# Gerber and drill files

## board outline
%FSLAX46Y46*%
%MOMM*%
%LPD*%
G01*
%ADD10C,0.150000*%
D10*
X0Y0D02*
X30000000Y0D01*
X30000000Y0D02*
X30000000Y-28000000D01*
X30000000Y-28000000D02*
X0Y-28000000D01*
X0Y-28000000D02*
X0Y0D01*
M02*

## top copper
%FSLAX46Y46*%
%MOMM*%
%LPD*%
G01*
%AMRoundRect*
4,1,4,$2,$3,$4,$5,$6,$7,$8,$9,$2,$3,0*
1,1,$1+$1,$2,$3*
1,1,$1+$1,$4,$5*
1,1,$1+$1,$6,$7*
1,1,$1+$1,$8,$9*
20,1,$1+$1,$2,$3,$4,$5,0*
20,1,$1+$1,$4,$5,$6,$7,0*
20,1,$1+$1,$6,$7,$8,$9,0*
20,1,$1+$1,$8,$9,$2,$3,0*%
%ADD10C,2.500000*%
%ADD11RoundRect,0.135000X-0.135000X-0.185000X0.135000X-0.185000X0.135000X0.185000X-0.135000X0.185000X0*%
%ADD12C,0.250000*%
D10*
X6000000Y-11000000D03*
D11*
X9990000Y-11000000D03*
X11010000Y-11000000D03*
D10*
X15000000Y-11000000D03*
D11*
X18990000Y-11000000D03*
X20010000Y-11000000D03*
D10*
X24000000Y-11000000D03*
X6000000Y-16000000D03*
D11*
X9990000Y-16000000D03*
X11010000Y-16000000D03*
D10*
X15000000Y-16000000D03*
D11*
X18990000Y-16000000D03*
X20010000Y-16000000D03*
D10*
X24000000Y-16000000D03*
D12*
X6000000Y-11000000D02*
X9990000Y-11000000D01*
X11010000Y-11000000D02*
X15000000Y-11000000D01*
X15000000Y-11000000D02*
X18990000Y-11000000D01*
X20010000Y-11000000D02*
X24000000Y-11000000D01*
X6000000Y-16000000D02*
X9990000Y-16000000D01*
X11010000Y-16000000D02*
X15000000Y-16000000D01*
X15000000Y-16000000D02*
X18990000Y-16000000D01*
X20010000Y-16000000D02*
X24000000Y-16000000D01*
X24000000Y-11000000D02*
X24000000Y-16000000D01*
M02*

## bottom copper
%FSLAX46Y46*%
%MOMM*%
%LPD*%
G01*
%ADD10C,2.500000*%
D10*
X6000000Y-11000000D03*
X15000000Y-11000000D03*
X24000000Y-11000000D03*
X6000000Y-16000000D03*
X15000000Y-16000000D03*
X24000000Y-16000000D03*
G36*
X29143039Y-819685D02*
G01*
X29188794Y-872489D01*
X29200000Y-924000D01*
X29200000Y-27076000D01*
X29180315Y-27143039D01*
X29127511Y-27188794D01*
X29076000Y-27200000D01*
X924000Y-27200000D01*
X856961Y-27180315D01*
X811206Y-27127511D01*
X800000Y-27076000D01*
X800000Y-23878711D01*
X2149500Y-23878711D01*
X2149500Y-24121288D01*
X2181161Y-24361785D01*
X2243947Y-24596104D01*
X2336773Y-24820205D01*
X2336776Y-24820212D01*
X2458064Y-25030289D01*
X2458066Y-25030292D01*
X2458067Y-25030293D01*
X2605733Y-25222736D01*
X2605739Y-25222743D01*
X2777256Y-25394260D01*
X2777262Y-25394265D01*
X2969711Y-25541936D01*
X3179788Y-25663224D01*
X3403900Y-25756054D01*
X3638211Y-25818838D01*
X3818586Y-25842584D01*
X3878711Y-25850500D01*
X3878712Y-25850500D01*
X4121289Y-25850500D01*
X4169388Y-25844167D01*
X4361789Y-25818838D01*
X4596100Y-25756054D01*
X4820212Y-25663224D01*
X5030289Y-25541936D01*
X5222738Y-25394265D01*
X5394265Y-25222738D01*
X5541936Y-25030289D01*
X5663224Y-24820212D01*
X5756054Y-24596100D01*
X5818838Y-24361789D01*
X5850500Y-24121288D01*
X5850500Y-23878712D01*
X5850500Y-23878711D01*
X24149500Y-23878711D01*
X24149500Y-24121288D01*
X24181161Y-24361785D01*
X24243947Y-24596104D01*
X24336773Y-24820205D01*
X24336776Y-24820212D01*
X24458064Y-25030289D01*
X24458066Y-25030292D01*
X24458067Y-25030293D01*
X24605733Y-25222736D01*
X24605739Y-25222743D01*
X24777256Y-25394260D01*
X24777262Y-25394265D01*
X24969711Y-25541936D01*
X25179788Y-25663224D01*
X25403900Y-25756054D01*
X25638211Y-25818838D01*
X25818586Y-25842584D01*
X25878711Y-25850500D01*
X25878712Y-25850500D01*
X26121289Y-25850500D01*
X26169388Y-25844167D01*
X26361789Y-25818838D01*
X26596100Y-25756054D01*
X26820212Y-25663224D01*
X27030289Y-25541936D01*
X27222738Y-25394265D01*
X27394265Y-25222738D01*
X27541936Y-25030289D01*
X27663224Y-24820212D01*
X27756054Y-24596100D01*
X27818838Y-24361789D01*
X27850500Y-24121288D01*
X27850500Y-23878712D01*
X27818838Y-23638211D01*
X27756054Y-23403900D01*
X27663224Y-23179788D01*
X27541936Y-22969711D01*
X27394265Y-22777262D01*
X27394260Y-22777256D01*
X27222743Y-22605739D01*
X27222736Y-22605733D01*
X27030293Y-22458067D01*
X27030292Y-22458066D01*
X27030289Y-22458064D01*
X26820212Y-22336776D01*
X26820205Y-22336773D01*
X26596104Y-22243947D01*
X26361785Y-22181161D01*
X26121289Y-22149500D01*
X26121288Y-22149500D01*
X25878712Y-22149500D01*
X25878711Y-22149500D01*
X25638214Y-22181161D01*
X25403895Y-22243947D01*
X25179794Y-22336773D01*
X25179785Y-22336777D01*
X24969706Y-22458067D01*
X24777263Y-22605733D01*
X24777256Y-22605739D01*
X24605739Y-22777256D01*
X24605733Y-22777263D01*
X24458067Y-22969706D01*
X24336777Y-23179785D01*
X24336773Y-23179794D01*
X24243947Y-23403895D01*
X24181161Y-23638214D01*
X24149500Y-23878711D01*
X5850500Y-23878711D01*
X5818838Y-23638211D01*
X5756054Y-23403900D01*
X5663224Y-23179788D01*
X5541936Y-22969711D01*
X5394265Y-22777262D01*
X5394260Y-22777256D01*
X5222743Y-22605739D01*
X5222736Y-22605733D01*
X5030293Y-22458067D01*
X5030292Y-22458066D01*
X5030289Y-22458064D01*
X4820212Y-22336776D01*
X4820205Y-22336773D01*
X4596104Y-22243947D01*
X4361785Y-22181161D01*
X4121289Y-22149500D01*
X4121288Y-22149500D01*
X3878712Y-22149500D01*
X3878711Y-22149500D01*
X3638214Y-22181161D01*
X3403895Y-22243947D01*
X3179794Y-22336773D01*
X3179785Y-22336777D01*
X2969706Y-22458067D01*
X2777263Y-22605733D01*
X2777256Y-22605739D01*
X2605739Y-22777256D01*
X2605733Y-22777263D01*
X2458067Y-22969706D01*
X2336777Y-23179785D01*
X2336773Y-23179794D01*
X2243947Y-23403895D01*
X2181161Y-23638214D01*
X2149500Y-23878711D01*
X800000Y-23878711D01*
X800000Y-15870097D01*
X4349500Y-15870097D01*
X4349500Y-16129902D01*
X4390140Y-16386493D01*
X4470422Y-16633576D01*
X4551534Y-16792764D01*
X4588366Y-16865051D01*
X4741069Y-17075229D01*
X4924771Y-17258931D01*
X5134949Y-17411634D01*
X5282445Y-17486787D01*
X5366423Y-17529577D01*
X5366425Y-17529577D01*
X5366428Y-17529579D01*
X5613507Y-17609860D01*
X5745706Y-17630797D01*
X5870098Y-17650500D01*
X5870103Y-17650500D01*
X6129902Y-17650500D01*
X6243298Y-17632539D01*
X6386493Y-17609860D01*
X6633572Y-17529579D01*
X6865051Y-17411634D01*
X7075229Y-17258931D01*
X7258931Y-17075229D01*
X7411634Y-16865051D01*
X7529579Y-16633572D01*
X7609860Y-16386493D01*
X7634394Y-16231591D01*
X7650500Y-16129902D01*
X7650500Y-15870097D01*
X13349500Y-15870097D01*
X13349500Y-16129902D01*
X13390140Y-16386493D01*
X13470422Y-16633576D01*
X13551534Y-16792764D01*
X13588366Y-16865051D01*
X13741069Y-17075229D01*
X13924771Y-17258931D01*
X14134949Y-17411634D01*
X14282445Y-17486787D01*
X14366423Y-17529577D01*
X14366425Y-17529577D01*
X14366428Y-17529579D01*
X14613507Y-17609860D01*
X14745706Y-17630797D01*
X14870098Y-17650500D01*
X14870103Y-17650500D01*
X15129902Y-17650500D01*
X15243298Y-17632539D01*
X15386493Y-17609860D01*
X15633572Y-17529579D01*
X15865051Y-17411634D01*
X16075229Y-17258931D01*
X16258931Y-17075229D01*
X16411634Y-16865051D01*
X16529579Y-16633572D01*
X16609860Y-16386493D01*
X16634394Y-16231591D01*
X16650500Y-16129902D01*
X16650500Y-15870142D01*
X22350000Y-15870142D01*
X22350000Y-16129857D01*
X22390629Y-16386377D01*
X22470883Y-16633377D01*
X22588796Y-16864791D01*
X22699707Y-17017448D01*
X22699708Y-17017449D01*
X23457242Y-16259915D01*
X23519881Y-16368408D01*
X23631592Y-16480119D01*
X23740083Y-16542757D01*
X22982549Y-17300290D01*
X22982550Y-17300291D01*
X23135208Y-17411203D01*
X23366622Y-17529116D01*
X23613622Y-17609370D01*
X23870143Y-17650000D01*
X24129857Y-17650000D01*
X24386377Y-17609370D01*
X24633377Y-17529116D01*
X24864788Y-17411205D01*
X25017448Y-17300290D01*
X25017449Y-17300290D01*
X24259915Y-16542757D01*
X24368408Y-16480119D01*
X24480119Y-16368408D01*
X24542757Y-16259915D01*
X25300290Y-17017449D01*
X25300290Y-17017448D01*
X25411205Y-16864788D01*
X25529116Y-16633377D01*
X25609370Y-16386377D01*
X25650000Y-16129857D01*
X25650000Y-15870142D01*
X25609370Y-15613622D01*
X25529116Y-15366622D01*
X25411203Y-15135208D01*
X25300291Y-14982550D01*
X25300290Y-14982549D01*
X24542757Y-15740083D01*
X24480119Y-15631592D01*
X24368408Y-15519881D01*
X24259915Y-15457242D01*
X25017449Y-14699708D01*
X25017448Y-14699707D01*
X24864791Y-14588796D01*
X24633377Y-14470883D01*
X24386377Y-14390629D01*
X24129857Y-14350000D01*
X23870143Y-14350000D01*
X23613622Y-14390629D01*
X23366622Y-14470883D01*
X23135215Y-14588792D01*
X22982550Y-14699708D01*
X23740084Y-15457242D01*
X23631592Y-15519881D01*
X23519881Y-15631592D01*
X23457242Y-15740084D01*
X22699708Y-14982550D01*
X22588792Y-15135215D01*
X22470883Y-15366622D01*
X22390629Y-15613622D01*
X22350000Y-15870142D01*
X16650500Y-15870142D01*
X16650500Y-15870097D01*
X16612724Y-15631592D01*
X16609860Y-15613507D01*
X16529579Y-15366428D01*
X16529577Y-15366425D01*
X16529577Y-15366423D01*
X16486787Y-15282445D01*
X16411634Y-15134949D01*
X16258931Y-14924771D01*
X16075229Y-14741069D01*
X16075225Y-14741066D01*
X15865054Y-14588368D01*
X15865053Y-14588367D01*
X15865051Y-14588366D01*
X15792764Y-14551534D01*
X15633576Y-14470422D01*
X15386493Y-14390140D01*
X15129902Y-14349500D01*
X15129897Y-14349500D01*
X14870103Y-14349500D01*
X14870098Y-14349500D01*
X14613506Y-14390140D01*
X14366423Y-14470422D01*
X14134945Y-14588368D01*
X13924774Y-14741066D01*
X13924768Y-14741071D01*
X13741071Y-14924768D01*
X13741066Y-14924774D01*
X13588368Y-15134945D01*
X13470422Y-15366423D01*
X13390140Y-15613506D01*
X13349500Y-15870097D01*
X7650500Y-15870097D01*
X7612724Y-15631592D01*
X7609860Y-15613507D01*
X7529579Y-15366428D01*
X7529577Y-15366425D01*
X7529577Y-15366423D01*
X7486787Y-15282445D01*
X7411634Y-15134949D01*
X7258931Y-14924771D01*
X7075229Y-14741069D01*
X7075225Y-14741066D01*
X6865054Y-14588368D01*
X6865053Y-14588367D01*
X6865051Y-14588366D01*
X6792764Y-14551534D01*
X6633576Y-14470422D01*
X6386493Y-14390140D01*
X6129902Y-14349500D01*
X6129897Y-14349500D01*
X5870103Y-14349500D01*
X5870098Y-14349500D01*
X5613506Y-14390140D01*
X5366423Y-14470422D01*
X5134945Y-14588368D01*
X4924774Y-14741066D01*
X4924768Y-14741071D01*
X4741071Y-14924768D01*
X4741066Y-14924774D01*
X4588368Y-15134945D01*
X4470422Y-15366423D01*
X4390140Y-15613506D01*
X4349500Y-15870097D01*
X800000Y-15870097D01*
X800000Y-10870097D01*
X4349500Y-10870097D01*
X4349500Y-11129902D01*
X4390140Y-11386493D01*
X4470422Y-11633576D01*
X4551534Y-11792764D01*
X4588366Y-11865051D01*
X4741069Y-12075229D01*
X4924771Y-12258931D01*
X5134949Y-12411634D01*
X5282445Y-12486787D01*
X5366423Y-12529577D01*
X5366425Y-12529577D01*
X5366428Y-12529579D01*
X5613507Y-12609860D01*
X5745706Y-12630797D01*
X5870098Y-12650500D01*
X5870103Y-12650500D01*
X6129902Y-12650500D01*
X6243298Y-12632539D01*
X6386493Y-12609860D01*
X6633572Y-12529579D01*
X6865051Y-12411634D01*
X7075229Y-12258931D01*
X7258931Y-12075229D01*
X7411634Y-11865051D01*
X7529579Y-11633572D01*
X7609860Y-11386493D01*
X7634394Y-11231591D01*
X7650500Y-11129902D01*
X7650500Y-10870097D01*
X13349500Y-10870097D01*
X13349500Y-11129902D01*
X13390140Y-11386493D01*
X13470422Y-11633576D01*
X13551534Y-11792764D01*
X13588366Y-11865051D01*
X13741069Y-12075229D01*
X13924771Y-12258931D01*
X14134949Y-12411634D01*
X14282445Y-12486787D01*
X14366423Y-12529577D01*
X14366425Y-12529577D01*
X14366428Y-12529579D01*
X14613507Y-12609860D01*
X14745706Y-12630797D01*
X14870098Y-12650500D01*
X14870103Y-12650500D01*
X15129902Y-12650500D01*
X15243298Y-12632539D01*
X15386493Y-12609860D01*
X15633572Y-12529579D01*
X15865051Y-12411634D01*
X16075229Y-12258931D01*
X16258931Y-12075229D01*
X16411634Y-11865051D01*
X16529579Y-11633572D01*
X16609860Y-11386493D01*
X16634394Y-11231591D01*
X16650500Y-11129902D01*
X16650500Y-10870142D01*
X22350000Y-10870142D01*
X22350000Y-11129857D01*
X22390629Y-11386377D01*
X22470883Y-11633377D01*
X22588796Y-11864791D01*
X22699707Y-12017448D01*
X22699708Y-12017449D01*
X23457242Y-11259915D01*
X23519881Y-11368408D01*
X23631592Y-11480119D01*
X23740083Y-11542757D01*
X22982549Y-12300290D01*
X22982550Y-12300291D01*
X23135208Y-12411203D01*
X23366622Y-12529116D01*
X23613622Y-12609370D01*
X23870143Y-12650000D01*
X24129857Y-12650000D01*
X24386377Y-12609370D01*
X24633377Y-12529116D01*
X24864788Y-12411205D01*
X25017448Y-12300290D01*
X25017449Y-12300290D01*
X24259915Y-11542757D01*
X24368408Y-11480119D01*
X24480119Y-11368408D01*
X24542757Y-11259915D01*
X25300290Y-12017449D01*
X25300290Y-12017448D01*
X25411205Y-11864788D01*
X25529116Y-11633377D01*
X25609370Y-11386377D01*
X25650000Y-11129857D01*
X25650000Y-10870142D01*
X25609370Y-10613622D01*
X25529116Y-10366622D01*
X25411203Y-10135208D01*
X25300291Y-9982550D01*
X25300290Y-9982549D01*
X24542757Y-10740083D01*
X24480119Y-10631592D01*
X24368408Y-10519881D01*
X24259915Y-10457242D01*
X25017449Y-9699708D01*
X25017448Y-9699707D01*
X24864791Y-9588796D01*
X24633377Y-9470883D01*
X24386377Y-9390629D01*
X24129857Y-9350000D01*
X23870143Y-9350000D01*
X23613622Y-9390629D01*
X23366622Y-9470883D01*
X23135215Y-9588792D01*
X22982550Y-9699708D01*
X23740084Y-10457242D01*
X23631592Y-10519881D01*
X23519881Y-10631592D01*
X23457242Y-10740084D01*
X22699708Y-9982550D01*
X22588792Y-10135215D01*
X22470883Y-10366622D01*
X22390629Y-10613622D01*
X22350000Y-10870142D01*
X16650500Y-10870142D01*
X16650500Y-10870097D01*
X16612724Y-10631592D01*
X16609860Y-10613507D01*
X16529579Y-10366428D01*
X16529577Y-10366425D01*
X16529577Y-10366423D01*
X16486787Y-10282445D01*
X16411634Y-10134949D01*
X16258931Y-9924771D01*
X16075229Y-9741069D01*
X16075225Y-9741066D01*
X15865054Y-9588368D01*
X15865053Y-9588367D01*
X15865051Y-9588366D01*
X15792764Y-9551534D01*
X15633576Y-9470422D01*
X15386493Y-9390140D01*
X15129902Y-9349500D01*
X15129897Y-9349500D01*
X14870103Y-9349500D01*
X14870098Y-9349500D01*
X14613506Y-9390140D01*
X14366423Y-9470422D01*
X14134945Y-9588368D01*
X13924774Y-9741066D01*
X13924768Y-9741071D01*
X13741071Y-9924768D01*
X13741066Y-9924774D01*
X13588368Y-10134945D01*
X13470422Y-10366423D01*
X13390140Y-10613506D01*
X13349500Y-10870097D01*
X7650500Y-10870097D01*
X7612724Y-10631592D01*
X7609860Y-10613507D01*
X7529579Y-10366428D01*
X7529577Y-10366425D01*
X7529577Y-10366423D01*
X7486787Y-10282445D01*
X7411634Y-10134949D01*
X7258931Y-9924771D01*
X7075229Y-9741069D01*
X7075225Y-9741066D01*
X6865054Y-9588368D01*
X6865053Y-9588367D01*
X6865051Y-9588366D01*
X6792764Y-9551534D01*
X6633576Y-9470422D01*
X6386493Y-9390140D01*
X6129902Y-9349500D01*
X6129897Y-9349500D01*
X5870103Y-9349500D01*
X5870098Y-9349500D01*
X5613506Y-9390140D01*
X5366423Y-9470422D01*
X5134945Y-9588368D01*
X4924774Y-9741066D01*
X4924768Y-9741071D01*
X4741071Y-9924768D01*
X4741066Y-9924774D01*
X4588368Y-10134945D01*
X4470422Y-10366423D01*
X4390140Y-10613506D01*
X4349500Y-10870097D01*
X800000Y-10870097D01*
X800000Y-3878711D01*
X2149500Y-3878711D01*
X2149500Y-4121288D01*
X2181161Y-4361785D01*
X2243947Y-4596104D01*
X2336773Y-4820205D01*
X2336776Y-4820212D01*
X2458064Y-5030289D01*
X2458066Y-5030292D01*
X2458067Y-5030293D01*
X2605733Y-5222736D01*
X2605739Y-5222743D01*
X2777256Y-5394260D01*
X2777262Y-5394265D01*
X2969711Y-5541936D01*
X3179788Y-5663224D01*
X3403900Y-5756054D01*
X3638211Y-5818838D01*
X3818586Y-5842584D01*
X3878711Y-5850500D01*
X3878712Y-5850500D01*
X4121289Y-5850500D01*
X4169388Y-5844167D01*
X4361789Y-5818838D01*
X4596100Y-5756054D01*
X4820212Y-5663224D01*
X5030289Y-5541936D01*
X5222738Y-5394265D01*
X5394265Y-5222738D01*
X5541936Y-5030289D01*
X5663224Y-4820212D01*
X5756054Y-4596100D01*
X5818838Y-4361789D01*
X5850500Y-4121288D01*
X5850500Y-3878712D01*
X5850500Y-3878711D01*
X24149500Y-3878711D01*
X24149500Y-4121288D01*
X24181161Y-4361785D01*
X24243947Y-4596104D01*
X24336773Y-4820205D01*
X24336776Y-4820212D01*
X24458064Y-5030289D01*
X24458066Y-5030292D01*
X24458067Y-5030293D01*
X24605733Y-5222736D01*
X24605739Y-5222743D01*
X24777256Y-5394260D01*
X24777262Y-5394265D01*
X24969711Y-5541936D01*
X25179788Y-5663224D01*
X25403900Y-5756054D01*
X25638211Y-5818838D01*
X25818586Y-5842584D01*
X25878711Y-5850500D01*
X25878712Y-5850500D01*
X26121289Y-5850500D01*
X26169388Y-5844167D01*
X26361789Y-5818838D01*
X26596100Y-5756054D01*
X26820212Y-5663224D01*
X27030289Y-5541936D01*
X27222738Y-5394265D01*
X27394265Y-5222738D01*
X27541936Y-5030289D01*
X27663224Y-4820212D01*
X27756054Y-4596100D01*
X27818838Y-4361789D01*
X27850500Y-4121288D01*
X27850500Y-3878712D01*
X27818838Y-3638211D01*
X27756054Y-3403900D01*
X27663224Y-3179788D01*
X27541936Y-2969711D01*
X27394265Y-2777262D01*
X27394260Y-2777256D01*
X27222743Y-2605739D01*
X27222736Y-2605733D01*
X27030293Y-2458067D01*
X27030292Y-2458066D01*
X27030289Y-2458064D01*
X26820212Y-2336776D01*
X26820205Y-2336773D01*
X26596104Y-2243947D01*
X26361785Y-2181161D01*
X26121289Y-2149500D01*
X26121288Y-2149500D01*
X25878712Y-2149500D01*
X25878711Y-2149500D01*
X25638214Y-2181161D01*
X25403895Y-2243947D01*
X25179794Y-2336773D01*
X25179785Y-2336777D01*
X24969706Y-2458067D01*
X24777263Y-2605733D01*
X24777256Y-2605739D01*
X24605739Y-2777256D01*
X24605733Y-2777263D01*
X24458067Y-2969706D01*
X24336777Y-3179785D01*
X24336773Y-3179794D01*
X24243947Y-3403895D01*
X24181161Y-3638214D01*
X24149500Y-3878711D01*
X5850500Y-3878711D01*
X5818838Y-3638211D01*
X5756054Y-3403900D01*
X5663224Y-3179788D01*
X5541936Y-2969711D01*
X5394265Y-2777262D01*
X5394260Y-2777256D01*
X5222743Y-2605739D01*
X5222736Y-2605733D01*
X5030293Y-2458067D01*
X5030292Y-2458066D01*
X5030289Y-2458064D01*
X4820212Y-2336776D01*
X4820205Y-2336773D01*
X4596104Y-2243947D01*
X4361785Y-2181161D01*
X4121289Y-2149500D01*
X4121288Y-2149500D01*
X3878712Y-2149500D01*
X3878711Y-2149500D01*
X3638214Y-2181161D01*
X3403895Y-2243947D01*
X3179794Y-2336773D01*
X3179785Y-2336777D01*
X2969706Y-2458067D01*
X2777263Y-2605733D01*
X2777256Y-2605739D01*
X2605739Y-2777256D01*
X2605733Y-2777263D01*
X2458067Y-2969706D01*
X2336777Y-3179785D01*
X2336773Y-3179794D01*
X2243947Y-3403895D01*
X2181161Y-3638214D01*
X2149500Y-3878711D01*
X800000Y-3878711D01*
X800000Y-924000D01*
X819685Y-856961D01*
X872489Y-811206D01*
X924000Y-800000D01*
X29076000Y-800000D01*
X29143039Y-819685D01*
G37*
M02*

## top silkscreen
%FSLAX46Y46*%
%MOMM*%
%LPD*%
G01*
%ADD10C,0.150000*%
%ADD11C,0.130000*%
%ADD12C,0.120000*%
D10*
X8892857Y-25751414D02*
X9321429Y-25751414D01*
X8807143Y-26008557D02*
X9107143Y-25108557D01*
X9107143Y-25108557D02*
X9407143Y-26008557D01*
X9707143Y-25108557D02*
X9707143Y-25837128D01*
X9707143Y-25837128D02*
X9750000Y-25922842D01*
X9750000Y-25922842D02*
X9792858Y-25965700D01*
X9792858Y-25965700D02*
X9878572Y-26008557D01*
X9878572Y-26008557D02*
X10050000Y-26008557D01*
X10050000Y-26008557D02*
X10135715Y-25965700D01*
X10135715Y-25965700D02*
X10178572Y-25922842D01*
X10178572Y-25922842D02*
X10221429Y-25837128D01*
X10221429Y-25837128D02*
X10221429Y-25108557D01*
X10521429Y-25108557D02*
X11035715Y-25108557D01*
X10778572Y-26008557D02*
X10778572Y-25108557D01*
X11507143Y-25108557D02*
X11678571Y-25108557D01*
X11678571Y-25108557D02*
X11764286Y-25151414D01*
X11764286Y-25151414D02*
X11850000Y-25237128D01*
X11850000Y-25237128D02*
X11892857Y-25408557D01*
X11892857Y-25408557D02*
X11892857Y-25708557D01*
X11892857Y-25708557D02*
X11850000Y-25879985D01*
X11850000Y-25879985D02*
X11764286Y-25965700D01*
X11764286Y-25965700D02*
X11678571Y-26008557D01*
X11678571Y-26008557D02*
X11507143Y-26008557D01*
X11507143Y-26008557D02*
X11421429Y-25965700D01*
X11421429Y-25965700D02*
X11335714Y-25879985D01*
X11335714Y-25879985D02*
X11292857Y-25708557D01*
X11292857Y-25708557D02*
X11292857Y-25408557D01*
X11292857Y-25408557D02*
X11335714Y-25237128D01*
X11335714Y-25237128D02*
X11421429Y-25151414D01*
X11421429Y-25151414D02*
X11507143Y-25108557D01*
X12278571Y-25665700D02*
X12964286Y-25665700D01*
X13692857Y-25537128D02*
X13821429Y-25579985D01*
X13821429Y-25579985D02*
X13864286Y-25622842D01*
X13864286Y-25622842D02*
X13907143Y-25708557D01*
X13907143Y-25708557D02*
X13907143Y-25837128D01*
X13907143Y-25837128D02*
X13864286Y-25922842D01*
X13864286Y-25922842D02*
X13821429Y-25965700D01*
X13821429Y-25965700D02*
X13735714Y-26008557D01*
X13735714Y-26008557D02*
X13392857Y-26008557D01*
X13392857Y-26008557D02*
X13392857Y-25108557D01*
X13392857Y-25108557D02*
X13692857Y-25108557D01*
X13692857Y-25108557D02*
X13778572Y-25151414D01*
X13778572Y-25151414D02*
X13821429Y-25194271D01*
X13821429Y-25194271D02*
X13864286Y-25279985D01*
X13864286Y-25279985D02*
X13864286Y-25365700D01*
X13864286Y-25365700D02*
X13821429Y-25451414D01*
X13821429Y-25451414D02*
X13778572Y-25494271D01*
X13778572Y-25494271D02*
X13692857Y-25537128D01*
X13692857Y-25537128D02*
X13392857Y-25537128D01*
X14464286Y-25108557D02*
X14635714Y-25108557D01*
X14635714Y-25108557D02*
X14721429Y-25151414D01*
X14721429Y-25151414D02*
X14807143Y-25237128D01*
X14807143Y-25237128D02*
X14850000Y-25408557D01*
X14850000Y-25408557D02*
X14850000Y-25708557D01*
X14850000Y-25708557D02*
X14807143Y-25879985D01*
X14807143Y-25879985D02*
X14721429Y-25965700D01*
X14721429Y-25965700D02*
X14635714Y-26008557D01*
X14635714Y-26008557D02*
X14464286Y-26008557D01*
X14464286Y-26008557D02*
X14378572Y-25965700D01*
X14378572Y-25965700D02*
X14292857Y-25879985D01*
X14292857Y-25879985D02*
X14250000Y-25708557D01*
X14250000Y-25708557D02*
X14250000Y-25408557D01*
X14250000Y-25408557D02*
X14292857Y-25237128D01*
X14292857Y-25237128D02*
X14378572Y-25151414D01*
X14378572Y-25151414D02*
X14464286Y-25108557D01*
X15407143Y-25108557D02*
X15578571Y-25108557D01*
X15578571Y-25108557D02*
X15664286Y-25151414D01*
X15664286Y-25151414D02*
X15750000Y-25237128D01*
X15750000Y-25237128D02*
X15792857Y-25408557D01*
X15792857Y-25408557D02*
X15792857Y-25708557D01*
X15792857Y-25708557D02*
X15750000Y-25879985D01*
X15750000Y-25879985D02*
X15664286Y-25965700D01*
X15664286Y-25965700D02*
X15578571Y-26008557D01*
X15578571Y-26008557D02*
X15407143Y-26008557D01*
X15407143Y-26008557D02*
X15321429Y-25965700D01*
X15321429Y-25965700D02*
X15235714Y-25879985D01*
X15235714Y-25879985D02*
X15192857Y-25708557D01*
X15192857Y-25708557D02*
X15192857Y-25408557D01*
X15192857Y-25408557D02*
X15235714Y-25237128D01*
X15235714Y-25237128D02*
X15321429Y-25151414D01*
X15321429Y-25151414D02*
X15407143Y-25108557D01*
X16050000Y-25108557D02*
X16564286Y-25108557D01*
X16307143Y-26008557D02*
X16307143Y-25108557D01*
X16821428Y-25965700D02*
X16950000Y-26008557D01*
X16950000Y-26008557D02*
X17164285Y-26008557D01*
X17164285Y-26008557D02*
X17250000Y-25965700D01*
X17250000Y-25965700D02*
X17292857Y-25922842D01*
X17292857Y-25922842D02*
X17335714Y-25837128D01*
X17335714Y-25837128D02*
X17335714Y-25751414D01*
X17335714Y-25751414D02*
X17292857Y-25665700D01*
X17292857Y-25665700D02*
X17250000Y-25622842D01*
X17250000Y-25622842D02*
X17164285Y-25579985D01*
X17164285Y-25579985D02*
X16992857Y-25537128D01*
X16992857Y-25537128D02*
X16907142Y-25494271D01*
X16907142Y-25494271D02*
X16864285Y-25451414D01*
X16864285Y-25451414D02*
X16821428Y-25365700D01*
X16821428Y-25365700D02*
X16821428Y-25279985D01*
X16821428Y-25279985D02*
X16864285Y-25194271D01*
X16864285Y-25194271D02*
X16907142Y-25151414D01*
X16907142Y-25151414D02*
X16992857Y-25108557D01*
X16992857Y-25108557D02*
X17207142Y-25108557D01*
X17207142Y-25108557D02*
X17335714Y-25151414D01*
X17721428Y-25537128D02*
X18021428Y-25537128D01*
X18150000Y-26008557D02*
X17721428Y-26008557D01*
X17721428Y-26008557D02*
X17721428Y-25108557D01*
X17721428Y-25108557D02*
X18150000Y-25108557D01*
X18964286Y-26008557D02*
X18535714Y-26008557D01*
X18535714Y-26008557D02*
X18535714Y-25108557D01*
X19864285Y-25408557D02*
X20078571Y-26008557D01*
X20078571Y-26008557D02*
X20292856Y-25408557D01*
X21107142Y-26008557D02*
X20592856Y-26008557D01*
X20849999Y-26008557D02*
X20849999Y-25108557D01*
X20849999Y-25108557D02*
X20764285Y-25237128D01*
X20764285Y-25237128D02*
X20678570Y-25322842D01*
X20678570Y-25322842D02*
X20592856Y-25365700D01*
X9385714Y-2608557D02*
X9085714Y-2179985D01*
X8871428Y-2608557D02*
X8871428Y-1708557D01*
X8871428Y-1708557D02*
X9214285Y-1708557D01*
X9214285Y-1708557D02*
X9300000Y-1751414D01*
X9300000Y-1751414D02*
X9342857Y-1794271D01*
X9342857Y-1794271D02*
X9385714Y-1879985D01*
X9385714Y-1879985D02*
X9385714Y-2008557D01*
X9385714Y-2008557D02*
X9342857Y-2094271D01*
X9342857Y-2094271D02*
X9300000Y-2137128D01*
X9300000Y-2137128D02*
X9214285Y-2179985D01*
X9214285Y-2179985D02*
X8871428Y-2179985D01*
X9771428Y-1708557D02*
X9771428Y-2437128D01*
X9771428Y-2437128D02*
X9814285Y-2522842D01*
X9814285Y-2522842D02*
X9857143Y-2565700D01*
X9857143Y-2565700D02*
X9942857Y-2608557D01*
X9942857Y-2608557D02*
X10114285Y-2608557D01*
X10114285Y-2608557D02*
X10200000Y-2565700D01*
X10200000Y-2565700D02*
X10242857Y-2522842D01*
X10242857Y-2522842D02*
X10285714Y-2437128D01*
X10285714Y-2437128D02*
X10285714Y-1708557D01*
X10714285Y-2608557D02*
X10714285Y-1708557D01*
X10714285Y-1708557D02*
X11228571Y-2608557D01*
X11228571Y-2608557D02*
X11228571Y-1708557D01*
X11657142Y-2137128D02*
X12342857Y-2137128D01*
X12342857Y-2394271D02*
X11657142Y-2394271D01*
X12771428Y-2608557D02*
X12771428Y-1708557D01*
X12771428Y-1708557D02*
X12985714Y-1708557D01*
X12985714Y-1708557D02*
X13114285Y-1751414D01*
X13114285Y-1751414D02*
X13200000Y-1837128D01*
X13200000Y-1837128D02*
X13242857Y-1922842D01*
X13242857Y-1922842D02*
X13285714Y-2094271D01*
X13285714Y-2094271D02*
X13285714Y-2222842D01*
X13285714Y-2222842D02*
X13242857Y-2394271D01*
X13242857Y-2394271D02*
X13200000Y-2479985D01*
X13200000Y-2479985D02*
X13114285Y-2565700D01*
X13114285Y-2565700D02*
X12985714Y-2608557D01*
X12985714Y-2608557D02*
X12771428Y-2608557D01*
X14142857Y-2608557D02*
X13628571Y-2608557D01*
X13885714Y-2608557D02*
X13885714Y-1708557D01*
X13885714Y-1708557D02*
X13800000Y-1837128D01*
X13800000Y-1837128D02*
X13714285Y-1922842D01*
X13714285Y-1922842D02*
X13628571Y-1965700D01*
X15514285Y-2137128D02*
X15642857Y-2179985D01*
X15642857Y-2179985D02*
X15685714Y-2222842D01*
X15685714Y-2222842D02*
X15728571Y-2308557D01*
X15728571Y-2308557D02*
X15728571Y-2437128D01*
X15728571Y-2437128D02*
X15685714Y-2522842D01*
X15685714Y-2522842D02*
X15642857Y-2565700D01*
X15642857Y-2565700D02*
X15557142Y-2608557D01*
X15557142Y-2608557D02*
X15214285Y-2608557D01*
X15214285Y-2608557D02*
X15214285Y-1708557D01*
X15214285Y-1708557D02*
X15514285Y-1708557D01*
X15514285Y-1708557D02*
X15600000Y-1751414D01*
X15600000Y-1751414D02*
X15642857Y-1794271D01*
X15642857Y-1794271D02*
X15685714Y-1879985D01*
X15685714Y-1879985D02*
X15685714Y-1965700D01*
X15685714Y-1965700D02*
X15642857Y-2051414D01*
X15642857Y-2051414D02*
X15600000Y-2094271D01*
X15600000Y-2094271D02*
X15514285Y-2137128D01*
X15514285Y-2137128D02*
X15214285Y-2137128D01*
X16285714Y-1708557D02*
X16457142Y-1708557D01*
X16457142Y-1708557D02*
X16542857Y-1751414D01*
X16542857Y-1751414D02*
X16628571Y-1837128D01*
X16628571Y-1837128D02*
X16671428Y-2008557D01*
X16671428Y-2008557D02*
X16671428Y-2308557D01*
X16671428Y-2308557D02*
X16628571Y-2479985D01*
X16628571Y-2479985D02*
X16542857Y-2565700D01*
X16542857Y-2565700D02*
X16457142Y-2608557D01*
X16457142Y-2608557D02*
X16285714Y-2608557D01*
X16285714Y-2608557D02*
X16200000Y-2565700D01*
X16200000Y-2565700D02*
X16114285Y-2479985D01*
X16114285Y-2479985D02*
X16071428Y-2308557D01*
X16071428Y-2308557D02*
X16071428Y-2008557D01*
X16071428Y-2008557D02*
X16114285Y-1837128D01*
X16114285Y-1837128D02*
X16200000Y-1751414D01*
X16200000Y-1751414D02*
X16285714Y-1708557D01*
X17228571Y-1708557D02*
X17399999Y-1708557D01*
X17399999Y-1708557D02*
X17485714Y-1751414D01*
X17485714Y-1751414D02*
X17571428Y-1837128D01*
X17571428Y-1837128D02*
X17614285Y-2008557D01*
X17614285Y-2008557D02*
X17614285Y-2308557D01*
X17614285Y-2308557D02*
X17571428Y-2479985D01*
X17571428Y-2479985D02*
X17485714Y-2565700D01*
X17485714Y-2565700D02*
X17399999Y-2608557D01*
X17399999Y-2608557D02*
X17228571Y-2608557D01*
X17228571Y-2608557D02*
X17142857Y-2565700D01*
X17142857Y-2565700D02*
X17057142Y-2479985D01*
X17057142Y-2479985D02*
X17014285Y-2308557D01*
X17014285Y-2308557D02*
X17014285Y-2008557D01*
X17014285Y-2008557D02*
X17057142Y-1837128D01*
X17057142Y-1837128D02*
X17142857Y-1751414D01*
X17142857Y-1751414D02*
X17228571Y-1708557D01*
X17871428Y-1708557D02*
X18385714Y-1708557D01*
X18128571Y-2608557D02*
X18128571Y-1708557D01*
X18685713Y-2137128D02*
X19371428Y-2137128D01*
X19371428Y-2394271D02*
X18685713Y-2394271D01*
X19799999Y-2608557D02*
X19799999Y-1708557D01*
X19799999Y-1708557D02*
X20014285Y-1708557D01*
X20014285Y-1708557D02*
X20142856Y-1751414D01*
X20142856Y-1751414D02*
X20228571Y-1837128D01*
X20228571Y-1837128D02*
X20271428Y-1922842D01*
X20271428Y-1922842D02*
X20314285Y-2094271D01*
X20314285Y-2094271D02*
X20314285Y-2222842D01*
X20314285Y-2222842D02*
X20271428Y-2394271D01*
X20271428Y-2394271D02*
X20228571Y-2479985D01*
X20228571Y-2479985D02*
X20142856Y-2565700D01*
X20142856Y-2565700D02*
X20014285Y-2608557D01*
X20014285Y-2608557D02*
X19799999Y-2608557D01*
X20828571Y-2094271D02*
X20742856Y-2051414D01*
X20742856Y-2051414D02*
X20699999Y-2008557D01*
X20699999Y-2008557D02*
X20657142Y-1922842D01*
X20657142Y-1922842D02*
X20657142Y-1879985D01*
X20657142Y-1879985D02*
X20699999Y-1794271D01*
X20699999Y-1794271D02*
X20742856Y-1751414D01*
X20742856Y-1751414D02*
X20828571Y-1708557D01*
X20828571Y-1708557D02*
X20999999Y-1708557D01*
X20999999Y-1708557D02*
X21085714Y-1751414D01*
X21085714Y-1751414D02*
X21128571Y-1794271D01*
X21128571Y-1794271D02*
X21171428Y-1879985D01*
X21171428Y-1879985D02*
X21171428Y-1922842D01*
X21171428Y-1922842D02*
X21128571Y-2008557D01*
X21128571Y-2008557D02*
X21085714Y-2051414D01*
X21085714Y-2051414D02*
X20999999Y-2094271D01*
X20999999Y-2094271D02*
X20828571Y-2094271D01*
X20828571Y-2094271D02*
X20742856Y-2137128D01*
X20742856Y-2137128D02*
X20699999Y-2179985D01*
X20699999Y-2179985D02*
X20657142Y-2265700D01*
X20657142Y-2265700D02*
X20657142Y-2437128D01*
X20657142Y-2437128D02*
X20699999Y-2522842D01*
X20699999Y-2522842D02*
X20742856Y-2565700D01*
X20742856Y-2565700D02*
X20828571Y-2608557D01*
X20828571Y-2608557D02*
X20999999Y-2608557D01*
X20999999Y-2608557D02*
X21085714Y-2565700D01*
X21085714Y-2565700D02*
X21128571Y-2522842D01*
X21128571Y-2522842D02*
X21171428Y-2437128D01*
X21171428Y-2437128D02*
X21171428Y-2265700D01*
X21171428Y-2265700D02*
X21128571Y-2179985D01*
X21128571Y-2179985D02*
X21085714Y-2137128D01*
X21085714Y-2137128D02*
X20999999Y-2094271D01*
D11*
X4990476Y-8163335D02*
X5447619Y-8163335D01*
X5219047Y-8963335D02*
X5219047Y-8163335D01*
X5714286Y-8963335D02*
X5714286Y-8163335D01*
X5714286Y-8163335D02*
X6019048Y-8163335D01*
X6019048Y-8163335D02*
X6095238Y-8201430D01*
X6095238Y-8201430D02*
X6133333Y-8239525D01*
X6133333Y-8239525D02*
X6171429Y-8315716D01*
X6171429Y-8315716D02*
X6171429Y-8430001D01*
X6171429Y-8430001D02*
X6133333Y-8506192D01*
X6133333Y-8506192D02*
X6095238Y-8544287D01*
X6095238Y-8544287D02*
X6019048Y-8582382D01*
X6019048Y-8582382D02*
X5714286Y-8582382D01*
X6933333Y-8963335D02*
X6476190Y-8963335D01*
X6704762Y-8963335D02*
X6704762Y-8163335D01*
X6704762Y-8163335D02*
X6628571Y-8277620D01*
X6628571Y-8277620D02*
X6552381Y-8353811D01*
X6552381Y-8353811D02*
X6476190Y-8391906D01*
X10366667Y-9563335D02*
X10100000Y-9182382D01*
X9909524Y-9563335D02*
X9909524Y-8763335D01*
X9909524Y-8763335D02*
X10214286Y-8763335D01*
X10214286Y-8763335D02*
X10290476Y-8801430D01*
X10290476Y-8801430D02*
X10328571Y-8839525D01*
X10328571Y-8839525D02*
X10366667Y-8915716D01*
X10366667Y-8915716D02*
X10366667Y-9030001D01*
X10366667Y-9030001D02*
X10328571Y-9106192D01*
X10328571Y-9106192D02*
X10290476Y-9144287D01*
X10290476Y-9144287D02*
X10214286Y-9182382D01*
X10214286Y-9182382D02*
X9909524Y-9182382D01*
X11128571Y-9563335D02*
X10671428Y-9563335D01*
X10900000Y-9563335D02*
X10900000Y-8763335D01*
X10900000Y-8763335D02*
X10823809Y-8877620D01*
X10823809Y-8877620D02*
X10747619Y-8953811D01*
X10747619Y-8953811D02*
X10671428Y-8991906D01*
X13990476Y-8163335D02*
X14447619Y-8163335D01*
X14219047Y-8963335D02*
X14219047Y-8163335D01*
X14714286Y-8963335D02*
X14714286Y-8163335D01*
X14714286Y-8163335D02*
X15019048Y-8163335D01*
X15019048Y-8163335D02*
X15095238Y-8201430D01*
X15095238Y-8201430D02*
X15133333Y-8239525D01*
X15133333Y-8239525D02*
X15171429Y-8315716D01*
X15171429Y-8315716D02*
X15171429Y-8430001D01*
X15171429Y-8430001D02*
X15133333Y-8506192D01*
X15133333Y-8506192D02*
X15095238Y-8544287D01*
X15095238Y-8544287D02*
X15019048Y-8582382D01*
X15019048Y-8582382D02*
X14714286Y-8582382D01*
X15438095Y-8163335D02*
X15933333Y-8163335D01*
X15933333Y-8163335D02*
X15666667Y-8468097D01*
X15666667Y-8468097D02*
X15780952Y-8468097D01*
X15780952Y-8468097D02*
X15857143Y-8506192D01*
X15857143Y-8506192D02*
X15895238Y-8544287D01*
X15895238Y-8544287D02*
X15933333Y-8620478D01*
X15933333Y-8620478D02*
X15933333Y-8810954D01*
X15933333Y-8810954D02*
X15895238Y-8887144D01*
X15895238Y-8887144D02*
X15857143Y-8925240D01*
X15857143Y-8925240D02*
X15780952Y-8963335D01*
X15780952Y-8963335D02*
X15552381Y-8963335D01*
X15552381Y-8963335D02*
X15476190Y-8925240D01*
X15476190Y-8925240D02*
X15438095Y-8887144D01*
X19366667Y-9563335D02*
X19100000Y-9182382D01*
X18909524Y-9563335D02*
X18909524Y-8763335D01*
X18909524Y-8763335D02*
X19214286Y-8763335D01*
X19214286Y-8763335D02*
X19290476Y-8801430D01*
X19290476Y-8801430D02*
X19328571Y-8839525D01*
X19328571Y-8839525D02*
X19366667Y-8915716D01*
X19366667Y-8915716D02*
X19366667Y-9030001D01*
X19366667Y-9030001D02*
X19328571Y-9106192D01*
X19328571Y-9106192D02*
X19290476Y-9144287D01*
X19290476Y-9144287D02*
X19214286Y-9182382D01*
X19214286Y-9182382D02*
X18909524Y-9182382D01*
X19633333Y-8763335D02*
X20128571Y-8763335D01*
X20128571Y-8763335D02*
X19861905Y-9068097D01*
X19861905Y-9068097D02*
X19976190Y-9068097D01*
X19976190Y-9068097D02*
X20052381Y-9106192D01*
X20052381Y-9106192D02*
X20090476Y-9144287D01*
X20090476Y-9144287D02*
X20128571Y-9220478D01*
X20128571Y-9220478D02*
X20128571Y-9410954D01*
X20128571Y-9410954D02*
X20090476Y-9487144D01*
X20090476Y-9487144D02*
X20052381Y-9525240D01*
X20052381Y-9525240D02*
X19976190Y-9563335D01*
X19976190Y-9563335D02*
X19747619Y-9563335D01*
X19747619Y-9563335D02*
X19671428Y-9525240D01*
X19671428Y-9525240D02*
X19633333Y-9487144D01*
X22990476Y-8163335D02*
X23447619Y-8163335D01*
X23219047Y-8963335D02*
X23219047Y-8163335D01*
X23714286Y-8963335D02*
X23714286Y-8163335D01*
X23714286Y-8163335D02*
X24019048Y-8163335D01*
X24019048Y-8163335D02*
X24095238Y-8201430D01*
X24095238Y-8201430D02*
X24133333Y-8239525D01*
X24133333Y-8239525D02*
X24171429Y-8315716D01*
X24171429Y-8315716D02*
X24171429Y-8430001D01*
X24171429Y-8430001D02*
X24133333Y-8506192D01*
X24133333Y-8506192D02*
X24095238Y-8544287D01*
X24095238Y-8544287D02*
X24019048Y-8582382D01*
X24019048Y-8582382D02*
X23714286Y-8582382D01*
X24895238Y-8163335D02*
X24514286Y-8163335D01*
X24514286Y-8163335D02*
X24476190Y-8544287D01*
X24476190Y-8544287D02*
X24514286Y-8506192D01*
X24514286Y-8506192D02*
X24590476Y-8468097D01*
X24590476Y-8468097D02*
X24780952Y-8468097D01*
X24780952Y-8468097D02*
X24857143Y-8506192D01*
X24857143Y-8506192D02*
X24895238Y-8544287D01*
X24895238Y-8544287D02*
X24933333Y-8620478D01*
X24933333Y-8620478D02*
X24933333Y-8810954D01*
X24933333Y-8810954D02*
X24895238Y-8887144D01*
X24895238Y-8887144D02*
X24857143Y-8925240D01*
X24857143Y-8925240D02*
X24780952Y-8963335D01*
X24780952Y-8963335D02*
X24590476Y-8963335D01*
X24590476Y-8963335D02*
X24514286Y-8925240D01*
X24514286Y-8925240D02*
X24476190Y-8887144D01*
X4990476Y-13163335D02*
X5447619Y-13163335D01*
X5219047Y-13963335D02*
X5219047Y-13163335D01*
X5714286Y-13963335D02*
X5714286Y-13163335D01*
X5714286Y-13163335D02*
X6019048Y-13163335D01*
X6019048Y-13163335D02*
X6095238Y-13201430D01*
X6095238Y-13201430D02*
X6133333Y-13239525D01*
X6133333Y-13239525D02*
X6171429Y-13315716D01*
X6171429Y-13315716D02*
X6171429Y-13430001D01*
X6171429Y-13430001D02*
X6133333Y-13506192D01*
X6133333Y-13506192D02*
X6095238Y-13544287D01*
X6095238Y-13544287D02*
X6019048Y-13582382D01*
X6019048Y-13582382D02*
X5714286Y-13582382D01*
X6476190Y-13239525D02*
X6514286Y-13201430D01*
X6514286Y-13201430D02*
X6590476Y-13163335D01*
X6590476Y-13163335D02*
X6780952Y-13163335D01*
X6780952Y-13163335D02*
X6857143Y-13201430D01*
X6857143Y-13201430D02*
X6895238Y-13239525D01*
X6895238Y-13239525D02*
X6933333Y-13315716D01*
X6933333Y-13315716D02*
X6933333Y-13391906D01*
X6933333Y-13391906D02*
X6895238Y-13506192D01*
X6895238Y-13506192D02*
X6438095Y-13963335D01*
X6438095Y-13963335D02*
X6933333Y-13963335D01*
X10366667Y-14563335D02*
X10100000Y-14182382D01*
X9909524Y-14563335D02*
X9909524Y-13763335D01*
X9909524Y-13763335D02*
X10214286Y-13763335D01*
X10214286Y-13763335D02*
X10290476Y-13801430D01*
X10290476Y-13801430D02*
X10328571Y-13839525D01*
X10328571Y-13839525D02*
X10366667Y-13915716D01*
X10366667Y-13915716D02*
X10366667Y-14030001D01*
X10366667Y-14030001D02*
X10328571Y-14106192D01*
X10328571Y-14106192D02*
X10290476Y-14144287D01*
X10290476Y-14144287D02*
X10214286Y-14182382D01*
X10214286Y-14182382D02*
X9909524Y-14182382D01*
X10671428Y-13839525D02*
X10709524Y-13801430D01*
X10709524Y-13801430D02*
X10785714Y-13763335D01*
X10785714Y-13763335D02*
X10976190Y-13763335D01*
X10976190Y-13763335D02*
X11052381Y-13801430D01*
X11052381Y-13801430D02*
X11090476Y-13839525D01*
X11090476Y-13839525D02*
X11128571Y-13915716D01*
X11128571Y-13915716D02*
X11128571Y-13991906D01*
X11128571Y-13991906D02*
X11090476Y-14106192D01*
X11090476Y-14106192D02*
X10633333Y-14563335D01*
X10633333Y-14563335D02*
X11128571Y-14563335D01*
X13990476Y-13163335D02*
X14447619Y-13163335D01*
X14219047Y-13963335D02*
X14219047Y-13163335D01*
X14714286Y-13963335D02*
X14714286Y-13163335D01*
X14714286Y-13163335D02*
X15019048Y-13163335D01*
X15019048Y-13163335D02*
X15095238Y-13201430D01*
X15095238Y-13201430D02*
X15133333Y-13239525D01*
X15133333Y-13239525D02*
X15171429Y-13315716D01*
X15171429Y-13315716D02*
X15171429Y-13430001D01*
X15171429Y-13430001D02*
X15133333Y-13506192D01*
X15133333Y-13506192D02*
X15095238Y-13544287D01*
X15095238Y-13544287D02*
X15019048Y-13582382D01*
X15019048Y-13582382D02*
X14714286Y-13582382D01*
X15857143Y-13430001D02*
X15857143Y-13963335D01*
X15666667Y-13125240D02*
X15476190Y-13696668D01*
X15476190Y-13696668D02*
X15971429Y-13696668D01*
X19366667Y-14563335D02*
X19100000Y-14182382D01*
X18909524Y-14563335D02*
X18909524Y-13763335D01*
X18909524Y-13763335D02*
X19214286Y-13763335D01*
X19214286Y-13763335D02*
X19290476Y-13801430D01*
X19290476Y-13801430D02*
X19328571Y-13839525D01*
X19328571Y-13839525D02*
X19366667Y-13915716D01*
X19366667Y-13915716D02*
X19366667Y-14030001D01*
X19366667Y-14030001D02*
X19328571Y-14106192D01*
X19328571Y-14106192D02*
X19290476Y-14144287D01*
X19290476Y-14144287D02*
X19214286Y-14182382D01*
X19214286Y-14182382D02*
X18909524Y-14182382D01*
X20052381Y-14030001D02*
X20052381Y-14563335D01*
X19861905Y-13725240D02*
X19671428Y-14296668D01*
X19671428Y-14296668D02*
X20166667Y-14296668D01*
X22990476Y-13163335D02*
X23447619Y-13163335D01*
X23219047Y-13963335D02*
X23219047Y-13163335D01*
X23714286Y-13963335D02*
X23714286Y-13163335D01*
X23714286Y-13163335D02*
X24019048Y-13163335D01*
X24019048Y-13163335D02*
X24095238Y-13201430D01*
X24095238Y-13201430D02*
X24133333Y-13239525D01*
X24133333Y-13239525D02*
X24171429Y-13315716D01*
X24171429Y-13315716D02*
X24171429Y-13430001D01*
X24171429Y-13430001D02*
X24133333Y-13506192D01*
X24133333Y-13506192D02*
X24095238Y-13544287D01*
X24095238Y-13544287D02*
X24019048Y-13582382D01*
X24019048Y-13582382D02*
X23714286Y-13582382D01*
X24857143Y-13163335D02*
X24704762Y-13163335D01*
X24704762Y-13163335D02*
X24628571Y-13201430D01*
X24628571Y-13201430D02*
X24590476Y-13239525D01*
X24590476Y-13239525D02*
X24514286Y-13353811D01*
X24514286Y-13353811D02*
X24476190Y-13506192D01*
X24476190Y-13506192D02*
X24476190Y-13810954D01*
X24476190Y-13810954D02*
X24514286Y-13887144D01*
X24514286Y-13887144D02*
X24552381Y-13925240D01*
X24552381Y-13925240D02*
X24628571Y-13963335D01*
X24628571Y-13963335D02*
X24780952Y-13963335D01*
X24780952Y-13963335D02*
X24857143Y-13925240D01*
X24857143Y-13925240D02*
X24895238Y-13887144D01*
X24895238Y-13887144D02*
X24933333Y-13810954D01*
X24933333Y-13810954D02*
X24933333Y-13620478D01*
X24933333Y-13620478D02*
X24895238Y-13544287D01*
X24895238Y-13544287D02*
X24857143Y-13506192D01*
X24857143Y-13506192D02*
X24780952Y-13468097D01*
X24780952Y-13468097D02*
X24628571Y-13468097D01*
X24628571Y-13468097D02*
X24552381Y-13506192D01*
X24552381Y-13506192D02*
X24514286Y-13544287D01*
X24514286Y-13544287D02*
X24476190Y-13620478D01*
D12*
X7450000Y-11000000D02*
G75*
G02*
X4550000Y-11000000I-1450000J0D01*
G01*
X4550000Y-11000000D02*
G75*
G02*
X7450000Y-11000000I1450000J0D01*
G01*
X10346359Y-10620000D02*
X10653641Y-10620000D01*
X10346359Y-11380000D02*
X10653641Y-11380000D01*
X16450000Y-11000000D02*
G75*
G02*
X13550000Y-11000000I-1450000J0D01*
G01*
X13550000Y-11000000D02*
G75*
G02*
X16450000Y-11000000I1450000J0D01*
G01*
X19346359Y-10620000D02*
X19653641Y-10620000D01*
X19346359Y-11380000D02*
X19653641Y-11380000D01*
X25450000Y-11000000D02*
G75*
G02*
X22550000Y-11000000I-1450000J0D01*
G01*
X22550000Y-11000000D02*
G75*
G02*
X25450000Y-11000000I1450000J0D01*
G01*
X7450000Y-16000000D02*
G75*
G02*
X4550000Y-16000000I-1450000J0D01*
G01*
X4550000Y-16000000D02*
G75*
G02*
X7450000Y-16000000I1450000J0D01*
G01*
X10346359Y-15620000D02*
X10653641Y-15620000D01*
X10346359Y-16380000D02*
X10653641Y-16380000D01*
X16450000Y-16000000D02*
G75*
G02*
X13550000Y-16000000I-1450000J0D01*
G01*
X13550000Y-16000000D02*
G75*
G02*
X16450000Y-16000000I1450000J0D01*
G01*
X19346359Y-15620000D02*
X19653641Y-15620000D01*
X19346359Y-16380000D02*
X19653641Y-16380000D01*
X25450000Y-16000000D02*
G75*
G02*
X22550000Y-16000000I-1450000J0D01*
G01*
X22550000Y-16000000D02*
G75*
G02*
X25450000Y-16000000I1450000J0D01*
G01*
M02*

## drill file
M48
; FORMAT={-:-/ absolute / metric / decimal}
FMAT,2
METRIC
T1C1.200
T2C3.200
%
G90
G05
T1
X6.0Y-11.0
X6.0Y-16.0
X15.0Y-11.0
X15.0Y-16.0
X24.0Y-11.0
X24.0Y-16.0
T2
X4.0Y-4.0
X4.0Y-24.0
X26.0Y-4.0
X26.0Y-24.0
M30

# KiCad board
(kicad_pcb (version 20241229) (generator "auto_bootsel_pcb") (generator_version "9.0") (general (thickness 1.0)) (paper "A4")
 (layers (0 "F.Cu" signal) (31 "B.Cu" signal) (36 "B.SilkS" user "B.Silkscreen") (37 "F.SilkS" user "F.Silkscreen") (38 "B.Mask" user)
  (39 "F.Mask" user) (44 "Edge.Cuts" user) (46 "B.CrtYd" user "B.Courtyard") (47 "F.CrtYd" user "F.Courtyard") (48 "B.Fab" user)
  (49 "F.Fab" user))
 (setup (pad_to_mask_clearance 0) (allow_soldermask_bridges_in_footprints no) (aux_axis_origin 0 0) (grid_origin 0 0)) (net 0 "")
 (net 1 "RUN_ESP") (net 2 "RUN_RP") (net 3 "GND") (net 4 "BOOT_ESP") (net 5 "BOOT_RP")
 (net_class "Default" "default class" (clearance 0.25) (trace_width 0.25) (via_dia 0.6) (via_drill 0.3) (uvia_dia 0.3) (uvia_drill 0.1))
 (gr_line (start 0 0) (end 30 0) (stroke (width 0.15) (type solid)) (layer "Edge.Cuts"))
 (gr_line (start 30 0) (end 30 28) (stroke (width 0.15) (type solid)) (layer "Edge.Cuts"))
 (gr_line (start 30 28) (end 0 28) (stroke (width 0.15) (type solid)) (layer "Edge.Cuts"))
 (gr_line (start 0 28) (end 0 0) (stroke (width 0.15) (type solid)) (layer "Edge.Cuts"))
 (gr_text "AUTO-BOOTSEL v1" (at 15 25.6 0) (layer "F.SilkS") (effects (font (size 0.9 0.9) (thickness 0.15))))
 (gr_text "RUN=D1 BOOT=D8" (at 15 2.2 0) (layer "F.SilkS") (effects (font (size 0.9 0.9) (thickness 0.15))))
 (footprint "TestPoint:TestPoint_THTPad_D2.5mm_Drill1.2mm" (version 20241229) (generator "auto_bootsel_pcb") (layer "F.Cu") (at 6 11 0)
  (fp_circle (center 0 0) (end 0 1.45) (stroke (width 0.12) (type solid)) (fill no) (layer "F.SilkS")) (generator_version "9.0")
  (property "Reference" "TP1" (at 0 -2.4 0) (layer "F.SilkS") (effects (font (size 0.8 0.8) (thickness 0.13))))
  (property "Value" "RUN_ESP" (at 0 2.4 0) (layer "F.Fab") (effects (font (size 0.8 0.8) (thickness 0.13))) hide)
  (pad 1 thru_hole circle (at 0 0) (size 2.5 2.5) (drill 1.2) (layers "*.Cu" "*.Mask") (remove_unused_layers no) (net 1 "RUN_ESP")))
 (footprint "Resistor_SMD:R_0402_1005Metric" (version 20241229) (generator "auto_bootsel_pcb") (layer "F.Cu") (at 10.5 11 0)
  (fp_line (start -0.153641 -0.38) (end 0.153641 -0.38) (stroke (width 0.12) (type solid)) (layer "F.SilkS"))
  (fp_line (start -0.153641 0.38) (end 0.153641 0.38) (stroke (width 0.12) (type solid)) (layer "F.SilkS"))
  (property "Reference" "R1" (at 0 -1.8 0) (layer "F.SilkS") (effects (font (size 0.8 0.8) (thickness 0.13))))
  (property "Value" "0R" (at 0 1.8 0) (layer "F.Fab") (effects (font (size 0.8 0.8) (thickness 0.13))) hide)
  (pad 1 smd roundrect (at -0.51 0) (size 0.54 0.64) (layers "F.Cu" "F.Mask" "F.Paste") (roundrect_rratio 0.25) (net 1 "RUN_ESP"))
  (pad 2 smd roundrect (at 0.51 0) (size 0.54 0.64) (layers "F.Cu" "F.Mask" "F.Paste") (roundrect_rratio 0.25) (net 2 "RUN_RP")))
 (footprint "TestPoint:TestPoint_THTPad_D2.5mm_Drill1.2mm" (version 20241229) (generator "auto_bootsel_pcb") (layer "F.Cu") (at 15 11 0)
  (fp_circle (center 0 0) (end 0 1.45) (stroke (width 0.12) (type solid)) (fill no) (layer "F.SilkS")) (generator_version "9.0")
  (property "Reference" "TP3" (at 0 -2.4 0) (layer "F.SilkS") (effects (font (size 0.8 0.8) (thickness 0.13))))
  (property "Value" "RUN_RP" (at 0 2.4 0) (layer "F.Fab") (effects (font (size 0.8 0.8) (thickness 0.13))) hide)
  (pad 1 thru_hole circle (at 0 0) (size 2.5 2.5) (drill 1.2) (layers "*.Cu" "*.Mask") (remove_unused_layers no) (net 2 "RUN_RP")))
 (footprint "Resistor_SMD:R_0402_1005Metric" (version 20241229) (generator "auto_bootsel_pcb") (layer "F.Cu") (at 19.5 11 0)
  (fp_line (start -0.153641 -0.38) (end 0.153641 -0.38) (stroke (width 0.12) (type solid)) (layer "F.SilkS"))
  (fp_line (start -0.153641 0.38) (end 0.153641 0.38) (stroke (width 0.12) (type solid)) (layer "F.SilkS"))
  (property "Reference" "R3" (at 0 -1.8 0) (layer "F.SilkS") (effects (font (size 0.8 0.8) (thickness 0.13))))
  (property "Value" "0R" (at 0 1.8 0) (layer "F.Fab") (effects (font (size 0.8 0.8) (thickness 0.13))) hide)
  (pad 1 smd roundrect (at -0.51 0) (size 0.54 0.64) (layers "F.Cu" "F.Mask" "F.Paste") (roundrect_rratio 0.25) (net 2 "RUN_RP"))
  (pad 2 smd roundrect (at 0.51 0) (size 0.54 0.64) (layers "F.Cu" "F.Mask" "F.Paste") (roundrect_rratio 0.25) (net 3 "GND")))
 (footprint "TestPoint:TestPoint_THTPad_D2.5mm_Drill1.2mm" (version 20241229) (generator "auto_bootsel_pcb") (layer "F.Cu") (at 24 11 0)
  (fp_circle (center 0 0) (end 0 1.45) (stroke (width 0.12) (type solid)) (fill no) (layer "F.SilkS")) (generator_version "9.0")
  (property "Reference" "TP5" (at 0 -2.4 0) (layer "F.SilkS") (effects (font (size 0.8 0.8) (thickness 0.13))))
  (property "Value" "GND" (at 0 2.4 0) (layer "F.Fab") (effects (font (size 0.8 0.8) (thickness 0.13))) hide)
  (pad 1 thru_hole circle (at 0 0) (size 2.5 2.5) (drill 1.2) (layers "*.Cu" "*.Mask") (remove_unused_layers no) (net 3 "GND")))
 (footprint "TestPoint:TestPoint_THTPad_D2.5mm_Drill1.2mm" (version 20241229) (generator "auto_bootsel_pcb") (layer "F.Cu") (at 6 16 0)
  (fp_circle (center 0 0) (end 0 1.45) (stroke (width 0.12) (type solid)) (fill no) (layer "F.SilkS")) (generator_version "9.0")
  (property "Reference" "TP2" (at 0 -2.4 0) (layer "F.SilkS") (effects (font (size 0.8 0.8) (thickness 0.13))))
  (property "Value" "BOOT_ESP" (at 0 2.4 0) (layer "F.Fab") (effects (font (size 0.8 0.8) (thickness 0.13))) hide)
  (pad 1 thru_hole circle (at 0 0) (size 2.5 2.5) (drill 1.2) (layers "*.Cu" "*.Mask") (remove_unused_layers no) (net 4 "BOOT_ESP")))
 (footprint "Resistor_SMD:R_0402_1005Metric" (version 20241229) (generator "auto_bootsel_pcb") (layer "F.Cu") (at 10.5 16 0)
  (fp_line (start -0.153641 -0.38) (end 0.153641 -0.38) (stroke (width 0.12) (type solid)) (layer "F.SilkS"))
  (fp_line (start -0.153641 0.38) (end 0.153641 0.38) (stroke (width 0.12) (type solid)) (layer "F.SilkS"))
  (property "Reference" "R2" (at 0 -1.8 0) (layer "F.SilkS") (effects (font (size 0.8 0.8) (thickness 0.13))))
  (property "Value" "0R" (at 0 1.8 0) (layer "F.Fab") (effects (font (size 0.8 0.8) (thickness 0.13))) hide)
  (pad 1 smd roundrect (at -0.51 0) (size 0.54 0.64) (layers "F.Cu" "F.Mask" "F.Paste") (roundrect_rratio 0.25) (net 4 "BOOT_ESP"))
  (pad 2 smd roundrect (at 0.51 0) (size 0.54 0.64) (layers "F.Cu" "F.Mask" "F.Paste") (roundrect_rratio 0.25) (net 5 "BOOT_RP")))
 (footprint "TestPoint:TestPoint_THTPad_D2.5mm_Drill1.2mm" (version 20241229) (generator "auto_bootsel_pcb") (layer "F.Cu") (at 15 16 0)
  (fp_circle (center 0 0) (end 0 1.45) (stroke (width 0.12) (type solid)) (fill no) (layer "F.SilkS")) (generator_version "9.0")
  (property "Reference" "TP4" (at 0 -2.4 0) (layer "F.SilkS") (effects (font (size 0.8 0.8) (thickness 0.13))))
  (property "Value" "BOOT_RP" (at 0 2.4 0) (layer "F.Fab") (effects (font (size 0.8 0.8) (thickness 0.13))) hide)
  (pad 1 thru_hole circle (at 0 0) (size 2.5 2.5) (drill 1.2) (layers "*.Cu" "*.Mask") (remove_unused_layers no) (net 5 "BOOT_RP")))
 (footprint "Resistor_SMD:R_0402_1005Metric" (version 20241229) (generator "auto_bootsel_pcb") (layer "F.Cu") (at 19.5 16 0)
  (fp_line (start -0.153641 -0.38) (end 0.153641 -0.38) (stroke (width 0.12) (type solid)) (layer "F.SilkS"))
  (fp_line (start -0.153641 0.38) (end 0.153641 0.38) (stroke (width 0.12) (type solid)) (layer "F.SilkS"))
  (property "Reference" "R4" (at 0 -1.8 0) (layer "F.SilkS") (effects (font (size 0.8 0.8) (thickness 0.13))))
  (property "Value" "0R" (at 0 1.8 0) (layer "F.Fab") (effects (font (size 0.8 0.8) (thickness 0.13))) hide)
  (pad 1 smd roundrect (at -0.51 0) (size 0.54 0.64) (layers "F.Cu" "F.Mask" "F.Paste") (roundrect_rratio 0.25) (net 5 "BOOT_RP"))
  (pad 2 smd roundrect (at 0.51 0) (size 0.54 0.64) (layers "F.Cu" "F.Mask" "F.Paste") (roundrect_rratio 0.25) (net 3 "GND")))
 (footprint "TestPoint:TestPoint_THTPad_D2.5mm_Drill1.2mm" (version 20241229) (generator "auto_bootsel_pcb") (layer "F.Cu") (at 24 16 0)
  (fp_circle (center 0 0) (end 0 1.45) (stroke (width 0.12) (type solid)) (fill no) (layer "F.SilkS")) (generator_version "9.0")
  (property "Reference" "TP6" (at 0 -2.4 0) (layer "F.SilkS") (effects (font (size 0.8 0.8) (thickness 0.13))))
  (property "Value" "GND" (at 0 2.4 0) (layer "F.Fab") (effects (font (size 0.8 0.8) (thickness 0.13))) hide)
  (pad 1 thru_hole circle (at 0 0) (size 2.5 2.5) (drill 1.2) (layers "*.Cu" "*.Mask") (remove_unused_layers no) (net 3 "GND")))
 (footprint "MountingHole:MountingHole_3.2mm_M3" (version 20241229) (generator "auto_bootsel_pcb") (layer "F.Cu") (at 4 4 0)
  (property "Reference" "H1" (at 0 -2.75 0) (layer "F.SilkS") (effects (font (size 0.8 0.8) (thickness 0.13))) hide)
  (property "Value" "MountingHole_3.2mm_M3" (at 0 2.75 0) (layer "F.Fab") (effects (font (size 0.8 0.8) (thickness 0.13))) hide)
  (pad "" np_thru_hole circle (at 0 0) (size 3.2 3.2) (drill 3.2) (layers "*.Cu" "*.Mask")))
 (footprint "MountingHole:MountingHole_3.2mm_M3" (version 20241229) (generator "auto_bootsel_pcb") (layer "F.Cu") (at 26 4 0)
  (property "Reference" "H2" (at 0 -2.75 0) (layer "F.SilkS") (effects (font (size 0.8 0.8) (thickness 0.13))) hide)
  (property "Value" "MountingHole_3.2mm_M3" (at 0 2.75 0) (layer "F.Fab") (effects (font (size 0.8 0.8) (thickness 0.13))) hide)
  (pad "" np_thru_hole circle (at 0 0) (size 3.2 3.2) (drill 3.2) (layers "*.Cu" "*.Mask")))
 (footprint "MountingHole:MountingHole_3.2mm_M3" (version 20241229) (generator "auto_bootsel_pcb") (layer "F.Cu") (at 4 24 0)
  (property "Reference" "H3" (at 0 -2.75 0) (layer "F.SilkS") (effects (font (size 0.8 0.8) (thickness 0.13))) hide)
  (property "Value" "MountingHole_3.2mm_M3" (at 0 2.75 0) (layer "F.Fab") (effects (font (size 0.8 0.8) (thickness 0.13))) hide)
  (pad "" np_thru_hole circle (at 0 0) (size 3.2 3.2) (drill 3.2) (layers "*.Cu" "*.Mask")))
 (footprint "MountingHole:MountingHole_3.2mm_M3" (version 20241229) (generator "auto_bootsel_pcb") (layer "F.Cu") (at 26 24 0)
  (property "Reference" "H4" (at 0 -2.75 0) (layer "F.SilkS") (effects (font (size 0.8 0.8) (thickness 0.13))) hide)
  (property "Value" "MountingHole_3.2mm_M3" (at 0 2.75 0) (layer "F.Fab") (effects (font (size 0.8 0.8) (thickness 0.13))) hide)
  (pad "" np_thru_hole circle (at 0 0) (size 3.2 3.2) (drill 3.2) (layers "*.Cu" "*.Mask")))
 (segment (start 6 11) (end 9.99 11) (width 0.25) (layer "F.Cu") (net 1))
 (segment (start 11.01 11) (end 15 11) (width 0.25) (layer "F.Cu") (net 2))
 (segment (start 15 11) (end 18.99 11) (width 0.25) (layer "F.Cu") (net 2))
 (segment (start 20.01 11) (end 24 11) (width 0.25) (layer "F.Cu") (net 3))
 (segment (start 6 16) (end 9.99 16) (width 0.25) (layer "F.Cu") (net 4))
 (segment (start 11.01 16) (end 15 16) (width 0.25) (layer "F.Cu") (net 5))
 (segment (start 15 16) (end 18.99 16) (width 0.25) (layer "F.Cu") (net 5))
 (segment (start 20.01 16) (end 24 16) (width 0.25) (layer "F.Cu") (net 3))
 (segment (start 24 11) (end 24 16) (width 0.25) (layer "F.Cu") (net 3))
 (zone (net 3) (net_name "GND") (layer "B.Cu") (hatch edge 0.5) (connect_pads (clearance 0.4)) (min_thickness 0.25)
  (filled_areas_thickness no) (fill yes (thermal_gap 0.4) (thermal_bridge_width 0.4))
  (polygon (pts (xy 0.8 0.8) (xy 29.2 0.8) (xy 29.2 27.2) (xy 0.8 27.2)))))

